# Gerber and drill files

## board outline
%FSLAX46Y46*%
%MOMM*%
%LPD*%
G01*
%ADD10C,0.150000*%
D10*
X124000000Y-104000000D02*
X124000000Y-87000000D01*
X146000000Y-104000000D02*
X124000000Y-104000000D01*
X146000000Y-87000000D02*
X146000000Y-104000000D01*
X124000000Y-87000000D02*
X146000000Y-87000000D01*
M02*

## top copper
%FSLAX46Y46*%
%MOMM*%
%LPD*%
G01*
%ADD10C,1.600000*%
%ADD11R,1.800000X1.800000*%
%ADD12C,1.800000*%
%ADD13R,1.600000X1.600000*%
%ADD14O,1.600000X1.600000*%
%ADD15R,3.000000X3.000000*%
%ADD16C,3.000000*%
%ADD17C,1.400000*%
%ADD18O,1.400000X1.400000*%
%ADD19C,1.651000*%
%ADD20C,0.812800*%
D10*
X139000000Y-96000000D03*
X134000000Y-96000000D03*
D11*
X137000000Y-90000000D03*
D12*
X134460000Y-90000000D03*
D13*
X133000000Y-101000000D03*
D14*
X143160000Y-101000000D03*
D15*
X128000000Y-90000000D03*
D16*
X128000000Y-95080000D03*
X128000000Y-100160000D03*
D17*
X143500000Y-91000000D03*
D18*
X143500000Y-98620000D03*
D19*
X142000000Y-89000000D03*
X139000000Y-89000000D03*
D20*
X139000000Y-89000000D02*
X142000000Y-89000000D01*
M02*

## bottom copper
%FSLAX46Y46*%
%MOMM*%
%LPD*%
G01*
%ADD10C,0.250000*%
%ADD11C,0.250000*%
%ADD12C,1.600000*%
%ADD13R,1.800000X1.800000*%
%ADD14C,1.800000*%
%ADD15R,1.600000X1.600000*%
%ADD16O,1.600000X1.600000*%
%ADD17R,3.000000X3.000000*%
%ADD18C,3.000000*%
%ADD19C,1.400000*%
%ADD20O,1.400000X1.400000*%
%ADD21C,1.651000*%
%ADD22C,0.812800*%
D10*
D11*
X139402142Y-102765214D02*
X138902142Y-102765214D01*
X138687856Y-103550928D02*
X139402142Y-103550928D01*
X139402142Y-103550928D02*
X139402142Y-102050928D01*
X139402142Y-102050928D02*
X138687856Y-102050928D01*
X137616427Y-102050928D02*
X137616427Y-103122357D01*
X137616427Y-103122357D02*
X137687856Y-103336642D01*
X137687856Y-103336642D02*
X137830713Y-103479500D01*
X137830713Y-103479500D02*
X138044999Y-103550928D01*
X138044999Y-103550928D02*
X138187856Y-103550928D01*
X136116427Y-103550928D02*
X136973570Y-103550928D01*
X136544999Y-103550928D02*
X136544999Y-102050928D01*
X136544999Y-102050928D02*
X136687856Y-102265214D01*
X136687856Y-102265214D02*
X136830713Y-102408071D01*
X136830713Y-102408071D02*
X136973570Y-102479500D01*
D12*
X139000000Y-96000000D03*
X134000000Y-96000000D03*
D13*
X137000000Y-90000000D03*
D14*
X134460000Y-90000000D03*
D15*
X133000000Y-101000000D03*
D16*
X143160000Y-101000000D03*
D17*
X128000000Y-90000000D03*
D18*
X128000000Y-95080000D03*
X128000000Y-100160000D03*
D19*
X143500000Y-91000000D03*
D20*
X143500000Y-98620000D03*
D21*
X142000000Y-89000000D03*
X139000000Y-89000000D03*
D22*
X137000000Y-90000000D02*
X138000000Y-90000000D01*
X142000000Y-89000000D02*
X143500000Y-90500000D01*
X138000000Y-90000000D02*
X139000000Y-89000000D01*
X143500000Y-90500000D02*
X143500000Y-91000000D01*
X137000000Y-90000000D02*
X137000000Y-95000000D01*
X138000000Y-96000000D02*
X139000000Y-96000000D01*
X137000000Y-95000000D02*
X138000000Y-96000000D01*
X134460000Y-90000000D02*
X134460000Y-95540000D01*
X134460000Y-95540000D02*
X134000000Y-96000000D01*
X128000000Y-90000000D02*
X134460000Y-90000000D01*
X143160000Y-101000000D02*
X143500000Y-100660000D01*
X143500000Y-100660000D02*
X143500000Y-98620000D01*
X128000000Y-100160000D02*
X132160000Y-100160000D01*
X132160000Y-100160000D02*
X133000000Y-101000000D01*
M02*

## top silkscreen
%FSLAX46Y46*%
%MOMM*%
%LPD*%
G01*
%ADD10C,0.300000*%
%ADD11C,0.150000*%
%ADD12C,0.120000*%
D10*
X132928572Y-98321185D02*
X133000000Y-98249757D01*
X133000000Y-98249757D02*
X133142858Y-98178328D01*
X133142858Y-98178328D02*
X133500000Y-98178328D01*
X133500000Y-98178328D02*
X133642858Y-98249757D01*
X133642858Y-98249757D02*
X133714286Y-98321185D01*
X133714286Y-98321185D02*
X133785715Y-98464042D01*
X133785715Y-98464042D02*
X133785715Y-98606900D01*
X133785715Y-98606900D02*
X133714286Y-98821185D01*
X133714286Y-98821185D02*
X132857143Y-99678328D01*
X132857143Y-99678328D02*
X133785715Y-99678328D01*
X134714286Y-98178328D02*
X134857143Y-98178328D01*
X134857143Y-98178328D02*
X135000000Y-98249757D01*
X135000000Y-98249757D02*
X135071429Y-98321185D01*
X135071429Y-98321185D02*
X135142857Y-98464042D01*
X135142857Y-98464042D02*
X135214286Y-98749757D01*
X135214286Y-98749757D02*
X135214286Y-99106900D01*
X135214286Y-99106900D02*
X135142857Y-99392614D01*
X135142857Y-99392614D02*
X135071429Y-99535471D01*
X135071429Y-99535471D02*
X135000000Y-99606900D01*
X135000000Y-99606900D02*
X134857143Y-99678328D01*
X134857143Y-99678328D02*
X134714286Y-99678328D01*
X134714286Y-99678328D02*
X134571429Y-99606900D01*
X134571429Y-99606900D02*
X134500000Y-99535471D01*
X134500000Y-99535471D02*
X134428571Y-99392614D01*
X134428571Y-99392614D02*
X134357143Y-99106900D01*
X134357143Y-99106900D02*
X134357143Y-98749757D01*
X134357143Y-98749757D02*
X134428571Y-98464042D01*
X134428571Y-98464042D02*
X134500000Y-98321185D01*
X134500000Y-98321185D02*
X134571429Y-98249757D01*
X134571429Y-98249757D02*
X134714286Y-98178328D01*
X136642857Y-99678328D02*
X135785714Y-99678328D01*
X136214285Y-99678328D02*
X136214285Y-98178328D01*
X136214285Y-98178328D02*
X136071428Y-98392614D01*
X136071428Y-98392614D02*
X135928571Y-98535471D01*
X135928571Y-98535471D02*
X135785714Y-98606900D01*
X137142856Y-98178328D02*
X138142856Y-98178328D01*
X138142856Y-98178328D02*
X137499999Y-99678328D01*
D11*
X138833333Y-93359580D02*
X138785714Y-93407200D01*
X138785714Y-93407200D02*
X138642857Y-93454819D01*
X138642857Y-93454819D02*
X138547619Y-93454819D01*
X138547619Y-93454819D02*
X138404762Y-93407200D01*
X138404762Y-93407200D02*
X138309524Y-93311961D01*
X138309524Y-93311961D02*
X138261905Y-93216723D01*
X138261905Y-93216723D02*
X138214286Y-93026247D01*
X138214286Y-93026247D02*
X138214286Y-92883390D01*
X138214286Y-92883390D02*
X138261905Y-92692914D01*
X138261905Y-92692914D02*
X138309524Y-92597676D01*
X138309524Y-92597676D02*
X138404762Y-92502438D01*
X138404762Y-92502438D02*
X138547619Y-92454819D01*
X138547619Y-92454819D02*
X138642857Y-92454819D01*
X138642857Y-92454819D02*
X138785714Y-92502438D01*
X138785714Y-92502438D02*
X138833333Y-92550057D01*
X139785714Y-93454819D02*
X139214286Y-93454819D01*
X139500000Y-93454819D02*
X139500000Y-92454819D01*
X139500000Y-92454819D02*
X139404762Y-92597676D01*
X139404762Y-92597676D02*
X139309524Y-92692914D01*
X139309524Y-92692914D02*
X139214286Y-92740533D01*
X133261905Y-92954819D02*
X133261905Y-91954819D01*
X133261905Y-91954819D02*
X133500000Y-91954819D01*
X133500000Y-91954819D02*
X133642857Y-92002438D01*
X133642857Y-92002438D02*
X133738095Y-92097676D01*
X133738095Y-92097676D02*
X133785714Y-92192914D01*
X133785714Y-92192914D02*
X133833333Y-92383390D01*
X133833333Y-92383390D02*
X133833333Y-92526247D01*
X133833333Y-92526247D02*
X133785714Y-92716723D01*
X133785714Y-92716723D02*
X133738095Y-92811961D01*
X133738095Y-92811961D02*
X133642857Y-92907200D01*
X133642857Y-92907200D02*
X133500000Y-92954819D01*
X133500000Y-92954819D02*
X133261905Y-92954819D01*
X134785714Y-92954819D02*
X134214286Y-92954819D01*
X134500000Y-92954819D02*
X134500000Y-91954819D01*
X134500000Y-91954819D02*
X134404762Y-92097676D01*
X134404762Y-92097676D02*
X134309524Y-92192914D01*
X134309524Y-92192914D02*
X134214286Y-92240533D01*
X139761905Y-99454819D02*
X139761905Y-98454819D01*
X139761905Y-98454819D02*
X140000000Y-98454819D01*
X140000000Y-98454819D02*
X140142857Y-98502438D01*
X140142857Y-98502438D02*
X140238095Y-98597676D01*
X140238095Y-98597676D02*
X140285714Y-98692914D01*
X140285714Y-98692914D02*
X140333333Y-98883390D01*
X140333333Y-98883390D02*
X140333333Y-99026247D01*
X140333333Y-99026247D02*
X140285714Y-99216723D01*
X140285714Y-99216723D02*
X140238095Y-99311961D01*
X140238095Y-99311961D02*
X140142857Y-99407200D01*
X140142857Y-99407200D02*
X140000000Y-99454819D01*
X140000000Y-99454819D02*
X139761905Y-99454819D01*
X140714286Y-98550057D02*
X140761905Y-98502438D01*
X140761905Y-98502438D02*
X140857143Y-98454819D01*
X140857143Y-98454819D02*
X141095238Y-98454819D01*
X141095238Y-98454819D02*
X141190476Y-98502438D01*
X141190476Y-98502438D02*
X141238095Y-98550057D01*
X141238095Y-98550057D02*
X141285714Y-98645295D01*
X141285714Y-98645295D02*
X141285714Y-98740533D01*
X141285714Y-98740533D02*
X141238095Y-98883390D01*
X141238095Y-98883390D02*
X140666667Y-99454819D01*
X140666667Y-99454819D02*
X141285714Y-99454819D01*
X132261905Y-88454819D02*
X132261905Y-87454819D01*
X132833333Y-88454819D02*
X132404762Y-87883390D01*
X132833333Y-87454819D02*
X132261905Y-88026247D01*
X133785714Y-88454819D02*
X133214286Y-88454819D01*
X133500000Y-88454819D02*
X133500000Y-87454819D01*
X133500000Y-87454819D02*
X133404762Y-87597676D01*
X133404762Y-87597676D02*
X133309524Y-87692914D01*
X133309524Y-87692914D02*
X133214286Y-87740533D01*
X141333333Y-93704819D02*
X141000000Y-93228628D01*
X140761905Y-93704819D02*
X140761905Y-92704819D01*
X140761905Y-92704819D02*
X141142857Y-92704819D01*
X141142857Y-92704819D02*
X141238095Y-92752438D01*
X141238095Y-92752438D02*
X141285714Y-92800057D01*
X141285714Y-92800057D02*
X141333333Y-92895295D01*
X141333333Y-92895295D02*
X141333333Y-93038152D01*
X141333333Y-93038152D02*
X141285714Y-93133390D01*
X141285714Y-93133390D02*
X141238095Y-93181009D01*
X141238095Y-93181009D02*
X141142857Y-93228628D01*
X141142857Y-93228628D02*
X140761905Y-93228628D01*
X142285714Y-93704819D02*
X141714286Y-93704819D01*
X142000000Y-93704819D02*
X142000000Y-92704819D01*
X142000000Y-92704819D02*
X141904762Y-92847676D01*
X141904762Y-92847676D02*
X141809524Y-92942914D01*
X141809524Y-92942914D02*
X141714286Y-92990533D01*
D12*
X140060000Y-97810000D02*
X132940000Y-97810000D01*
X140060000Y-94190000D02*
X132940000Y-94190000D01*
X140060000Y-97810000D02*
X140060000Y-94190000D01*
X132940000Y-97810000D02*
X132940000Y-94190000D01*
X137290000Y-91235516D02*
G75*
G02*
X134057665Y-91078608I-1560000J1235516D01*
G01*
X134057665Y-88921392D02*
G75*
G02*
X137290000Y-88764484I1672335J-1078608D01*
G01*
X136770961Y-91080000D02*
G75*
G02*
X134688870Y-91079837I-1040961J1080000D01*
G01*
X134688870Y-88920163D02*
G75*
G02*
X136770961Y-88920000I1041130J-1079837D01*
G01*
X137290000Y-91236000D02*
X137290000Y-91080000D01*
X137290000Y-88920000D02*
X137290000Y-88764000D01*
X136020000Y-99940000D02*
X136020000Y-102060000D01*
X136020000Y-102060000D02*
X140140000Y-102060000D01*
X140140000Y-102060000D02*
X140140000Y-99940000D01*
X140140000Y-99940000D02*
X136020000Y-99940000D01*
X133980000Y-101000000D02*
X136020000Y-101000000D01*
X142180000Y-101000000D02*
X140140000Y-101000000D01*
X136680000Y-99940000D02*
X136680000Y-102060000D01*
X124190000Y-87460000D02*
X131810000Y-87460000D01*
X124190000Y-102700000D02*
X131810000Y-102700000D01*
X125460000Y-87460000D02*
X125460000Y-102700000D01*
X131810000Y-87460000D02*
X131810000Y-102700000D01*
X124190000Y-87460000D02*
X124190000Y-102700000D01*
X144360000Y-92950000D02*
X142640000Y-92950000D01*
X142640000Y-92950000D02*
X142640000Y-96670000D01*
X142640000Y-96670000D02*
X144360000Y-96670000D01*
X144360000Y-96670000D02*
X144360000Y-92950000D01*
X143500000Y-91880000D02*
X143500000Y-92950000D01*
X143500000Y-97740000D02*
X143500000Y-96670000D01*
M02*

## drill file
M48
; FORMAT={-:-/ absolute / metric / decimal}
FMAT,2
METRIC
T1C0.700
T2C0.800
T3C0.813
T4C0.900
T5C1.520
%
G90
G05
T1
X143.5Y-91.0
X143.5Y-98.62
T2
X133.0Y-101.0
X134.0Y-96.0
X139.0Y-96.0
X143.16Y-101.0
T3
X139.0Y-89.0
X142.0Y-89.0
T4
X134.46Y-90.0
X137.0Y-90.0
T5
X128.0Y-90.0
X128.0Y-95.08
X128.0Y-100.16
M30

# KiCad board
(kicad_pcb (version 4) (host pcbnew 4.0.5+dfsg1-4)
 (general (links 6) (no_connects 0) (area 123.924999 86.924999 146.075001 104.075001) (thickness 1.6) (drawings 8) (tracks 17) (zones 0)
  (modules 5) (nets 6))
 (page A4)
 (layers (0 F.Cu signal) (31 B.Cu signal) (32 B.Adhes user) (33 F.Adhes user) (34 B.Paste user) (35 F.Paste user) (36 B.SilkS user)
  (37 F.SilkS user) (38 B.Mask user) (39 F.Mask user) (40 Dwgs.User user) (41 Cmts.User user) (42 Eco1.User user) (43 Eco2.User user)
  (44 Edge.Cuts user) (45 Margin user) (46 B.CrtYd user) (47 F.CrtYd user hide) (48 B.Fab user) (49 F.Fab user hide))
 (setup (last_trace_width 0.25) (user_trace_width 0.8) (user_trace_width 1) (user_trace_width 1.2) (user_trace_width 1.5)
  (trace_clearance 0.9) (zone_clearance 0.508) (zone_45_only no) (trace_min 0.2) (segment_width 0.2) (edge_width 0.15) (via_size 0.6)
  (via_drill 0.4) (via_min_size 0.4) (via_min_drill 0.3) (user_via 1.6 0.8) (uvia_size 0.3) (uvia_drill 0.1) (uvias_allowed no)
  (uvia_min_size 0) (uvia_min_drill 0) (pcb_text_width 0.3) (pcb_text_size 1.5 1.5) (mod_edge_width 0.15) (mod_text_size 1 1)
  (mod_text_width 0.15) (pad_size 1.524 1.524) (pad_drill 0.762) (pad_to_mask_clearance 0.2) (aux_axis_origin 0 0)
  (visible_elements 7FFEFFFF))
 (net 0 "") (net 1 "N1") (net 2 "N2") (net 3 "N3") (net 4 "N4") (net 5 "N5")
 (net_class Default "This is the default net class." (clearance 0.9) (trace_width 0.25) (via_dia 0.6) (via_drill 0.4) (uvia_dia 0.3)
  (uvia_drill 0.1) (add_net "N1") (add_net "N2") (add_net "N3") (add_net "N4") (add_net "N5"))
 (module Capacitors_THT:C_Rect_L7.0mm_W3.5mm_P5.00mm (layer F.Cu) (at 139 96 180)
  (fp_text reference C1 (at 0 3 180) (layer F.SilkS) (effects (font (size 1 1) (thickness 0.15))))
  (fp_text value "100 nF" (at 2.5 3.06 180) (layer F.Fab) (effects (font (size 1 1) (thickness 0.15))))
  (fp_line (start -1.06 -1.81) (end 6.06 -1.81) (layer F.SilkS) (width 0.12))
  (fp_line (start -1.06 1.81) (end 6.06 1.81) (layer F.SilkS) (width 0.12))
  (fp_line (start -1.06 -1.81) (end -1.06 1.81) (layer F.SilkS) (width 0.12))
  (fp_line (start 6.06 -1.81) (end 6.06 1.81) (layer F.SilkS) (width 0.12))
  (pad 1 thru_hole circle (at 0 0 180) (size 1.6 1.6) (drill 0.8) (layers *.Cu *.Mask) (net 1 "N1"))
  (pad 2 thru_hole circle (at 5 0 180) (size 1.6 1.6) (drill 0.8) (layers *.Cu *.Mask) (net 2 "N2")))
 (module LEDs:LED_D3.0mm (layer F.Cu) (at 137 90 180)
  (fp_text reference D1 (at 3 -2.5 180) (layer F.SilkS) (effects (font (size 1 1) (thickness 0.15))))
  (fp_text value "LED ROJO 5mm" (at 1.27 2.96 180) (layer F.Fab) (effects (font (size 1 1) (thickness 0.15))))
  (fp_arc (start 1.27 0) (end -0.29 -1.235516) (angle 108.8) (layer F.SilkS) (width 0.12))
  (fp_arc (start 1.27 0) (end -0.29 1.235516) (angle -108.8) (layer F.SilkS) (width 0.12))
  (fp_arc (start 1.27 0) (end 0.229039 -1.08) (angle 87.9) (layer F.SilkS) (width 0.12))
  (fp_arc (start 1.27 0) (end 0.229039 1.08) (angle -87.9) (layer F.SilkS) (width 0.12))
  (fp_line (start -0.29 -1.236) (end -0.29 -1.08) (layer F.SilkS) (width 0.12))
  (fp_line (start -0.29 1.08) (end -0.29 1.236) (layer F.SilkS) (width 0.12))
  (pad 1 thru_hole rect (at 0 0 180) (size 1.8 1.8) (drill 0.9) (layers *.Cu *.Mask) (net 1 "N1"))
  (pad 2 thru_hole circle (at 2.54 0 180) (size 1.8 1.8) (drill 0.9) (layers *.Cu *.Mask) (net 2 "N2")))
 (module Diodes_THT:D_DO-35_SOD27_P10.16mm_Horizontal (layer F.Cu) (at 133 101)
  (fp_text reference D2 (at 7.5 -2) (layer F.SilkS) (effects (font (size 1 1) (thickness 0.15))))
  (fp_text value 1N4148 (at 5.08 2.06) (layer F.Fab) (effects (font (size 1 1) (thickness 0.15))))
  (fp_line (start 3.02 -1.06) (end 3.02 1.06) (layer F.SilkS) (width 0.12))
  (fp_line (start 3.02 1.06) (end 7.14 1.06) (layer F.SilkS) (width 0.12))
  (fp_line (start 7.14 1.06) (end 7.14 -1.06) (layer F.SilkS) (width 0.12))
  (fp_line (start 7.14 -1.06) (end 3.02 -1.06) (layer F.SilkS) (width 0.12))
  (fp_line (start 0.98 0) (end 3.02 0) (layer F.SilkS) (width 0.12))
  (fp_line (start 9.18 0) (end 7.14 0) (layer F.SilkS) (width 0.12))
  (fp_line (start 3.68 -1.06) (end 3.68 1.06) (layer F.SilkS) (width 0.12))
  (pad 1 thru_hole rect (at 0 0) (size 1.6 1.6) (drill 0.8) (layers *.Cu *.Mask) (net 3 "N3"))
  (pad 2 thru_hole oval (at 10.16 0) (size 1.6 1.6) (drill 0.8) (layers *.Cu *.Mask) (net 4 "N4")))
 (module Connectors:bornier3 (layer F.Cu) (at 128 90 270)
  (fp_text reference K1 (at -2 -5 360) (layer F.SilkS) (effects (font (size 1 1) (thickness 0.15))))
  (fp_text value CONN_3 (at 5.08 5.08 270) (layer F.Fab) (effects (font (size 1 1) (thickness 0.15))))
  (fp_line (start -2.54 3.81) (end -2.54 -3.81) (layer F.SilkS) (width 0.12))
  (fp_line (start 12.7 3.81) (end 12.7 -3.81) (layer F.SilkS) (width 0.12))
  (fp_line (start -2.54 2.54) (end 12.7 2.54) (layer F.SilkS) (width 0.12))
  (fp_line (start -2.54 -3.81) (end 12.7 -3.81) (layer F.SilkS) (width 0.12))
  (fp_line (start -2.54 3.81) (end 12.7 3.81) (layer F.SilkS) (width 0.12))
  (pad 1 thru_hole rect (at 0 0 270) (size 3 3) (drill 1.52) (layers *.Cu *.Mask) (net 2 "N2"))
  (pad 2 thru_hole circle (at 5.08 0 270) (size 3 3) (drill 1.52) (layers *.Cu *.Mask) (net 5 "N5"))
  (pad 3 thru_hole circle (at 10.16 0 270) (size 3 3) (drill 1.52) (layers *.Cu *.Mask) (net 3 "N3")))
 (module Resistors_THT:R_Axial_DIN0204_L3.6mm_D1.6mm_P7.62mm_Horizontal (layer F.Cu) (at 143.5 91 270)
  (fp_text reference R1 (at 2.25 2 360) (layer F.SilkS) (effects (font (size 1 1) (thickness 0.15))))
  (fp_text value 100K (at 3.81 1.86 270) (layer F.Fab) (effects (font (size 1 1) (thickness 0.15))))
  (fp_line (start 1.95 -0.86) (end 1.95 0.86) (layer F.SilkS) (width 0.12))
  (fp_line (start 1.95 0.86) (end 5.67 0.86) (layer F.SilkS) (width 0.12))
  (fp_line (start 5.67 0.86) (end 5.67 -0.86) (layer F.SilkS) (width 0.12))
  (fp_line (start 5.67 -0.86) (end 1.95 -0.86) (layer F.SilkS) (width 0.12))
  (fp_line (start 0.88 0) (end 1.95 0) (layer F.SilkS) (width 0.12))
  (fp_line (start 6.74 0) (end 5.67 0) (layer F.SilkS) (width 0.12))
  (pad 1 thru_hole circle (at 0 0 270) (size 1.4 1.4) (drill 0.7) (layers *.Cu *.Mask) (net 1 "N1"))
  (pad 2 thru_hole oval (at 7.62 0 270) (size 1.4 1.4) (drill 0.7) (layers *.Cu *.Mask) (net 4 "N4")))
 (gr_line (start 124 104) (end 124 87) (angle 90) (layer Edge.Cuts) (width 0.15))
 (gr_line (start 146 104) (end 124 104) (angle 90) (layer Edge.Cuts) (width 0.15))
 (gr_line (start 146 87) (end 146 104) (angle 90) (layer Edge.Cuts) (width 0.15))
 (gr_line (start 124 87) (end 146 87) (angle 90) (layer Edge.Cuts) (width 0.15))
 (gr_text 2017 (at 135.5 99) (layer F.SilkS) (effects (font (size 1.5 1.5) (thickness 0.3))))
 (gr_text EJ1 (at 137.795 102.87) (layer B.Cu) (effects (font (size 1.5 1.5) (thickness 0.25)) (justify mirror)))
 (segment (start 137 90) (end 138 90) (width 0.8128) (layer B.Cu) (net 1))
 (segment (start 142 89) (end 143.5 90.5) (width 0.8128) (layer B.Cu) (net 1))
 (via (at 142 89) (size 1.651) (drill 0.8128) (layers F.Cu B.Cu) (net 1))
 (segment (start 139 89) (end 142 89) (width 0.8128) (layer F.Cu) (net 1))
 (via (at 139 89) (size 1.651) (drill 0.8128) (layers F.Cu B.Cu) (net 1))
 (segment (start 138 90) (end 139 89) (width 0.8128) (layer B.Cu) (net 1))
 (segment (start 143.5 90.5) (end 143.5 91) (width 0.8128) (layer B.Cu) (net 1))
 (segment (start 137 90) (end 137 95) (width 0.8128) (layer B.Cu) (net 1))
 (segment (start 138 96) (end 139 96) (width 0.8128) (layer B.Cu) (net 1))
 (segment (start 137 95) (end 138 96) (width 0.8128) (layer B.Cu) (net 1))
 (segment (start 134.46 90) (end 134.46 95.54) (width 0.8128) (layer B.Cu) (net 2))
 (segment (start 134.46 95.54) (end 134 96) (width 0.8128) (layer B.Cu) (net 2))
 (segment (start 128 90) (end 134.46 90) (width 0.8128) (layer B.Cu) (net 2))
 (segment (start 143.16 101) (end 143.5 100.66) (width 0.8128) (layer B.Cu) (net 4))
 (segment (start 143.5 100.66) (end 143.5 98.62) (width 0.8128) (layer B.Cu) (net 4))
 (segment (start 128 100.16) (end 132.16 100.16) (width 0.8128) (layer B.Cu) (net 3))
 (segment (start 132.16 100.16) (end 133 101) (width 0.8128) (layer B.Cu) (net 3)))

